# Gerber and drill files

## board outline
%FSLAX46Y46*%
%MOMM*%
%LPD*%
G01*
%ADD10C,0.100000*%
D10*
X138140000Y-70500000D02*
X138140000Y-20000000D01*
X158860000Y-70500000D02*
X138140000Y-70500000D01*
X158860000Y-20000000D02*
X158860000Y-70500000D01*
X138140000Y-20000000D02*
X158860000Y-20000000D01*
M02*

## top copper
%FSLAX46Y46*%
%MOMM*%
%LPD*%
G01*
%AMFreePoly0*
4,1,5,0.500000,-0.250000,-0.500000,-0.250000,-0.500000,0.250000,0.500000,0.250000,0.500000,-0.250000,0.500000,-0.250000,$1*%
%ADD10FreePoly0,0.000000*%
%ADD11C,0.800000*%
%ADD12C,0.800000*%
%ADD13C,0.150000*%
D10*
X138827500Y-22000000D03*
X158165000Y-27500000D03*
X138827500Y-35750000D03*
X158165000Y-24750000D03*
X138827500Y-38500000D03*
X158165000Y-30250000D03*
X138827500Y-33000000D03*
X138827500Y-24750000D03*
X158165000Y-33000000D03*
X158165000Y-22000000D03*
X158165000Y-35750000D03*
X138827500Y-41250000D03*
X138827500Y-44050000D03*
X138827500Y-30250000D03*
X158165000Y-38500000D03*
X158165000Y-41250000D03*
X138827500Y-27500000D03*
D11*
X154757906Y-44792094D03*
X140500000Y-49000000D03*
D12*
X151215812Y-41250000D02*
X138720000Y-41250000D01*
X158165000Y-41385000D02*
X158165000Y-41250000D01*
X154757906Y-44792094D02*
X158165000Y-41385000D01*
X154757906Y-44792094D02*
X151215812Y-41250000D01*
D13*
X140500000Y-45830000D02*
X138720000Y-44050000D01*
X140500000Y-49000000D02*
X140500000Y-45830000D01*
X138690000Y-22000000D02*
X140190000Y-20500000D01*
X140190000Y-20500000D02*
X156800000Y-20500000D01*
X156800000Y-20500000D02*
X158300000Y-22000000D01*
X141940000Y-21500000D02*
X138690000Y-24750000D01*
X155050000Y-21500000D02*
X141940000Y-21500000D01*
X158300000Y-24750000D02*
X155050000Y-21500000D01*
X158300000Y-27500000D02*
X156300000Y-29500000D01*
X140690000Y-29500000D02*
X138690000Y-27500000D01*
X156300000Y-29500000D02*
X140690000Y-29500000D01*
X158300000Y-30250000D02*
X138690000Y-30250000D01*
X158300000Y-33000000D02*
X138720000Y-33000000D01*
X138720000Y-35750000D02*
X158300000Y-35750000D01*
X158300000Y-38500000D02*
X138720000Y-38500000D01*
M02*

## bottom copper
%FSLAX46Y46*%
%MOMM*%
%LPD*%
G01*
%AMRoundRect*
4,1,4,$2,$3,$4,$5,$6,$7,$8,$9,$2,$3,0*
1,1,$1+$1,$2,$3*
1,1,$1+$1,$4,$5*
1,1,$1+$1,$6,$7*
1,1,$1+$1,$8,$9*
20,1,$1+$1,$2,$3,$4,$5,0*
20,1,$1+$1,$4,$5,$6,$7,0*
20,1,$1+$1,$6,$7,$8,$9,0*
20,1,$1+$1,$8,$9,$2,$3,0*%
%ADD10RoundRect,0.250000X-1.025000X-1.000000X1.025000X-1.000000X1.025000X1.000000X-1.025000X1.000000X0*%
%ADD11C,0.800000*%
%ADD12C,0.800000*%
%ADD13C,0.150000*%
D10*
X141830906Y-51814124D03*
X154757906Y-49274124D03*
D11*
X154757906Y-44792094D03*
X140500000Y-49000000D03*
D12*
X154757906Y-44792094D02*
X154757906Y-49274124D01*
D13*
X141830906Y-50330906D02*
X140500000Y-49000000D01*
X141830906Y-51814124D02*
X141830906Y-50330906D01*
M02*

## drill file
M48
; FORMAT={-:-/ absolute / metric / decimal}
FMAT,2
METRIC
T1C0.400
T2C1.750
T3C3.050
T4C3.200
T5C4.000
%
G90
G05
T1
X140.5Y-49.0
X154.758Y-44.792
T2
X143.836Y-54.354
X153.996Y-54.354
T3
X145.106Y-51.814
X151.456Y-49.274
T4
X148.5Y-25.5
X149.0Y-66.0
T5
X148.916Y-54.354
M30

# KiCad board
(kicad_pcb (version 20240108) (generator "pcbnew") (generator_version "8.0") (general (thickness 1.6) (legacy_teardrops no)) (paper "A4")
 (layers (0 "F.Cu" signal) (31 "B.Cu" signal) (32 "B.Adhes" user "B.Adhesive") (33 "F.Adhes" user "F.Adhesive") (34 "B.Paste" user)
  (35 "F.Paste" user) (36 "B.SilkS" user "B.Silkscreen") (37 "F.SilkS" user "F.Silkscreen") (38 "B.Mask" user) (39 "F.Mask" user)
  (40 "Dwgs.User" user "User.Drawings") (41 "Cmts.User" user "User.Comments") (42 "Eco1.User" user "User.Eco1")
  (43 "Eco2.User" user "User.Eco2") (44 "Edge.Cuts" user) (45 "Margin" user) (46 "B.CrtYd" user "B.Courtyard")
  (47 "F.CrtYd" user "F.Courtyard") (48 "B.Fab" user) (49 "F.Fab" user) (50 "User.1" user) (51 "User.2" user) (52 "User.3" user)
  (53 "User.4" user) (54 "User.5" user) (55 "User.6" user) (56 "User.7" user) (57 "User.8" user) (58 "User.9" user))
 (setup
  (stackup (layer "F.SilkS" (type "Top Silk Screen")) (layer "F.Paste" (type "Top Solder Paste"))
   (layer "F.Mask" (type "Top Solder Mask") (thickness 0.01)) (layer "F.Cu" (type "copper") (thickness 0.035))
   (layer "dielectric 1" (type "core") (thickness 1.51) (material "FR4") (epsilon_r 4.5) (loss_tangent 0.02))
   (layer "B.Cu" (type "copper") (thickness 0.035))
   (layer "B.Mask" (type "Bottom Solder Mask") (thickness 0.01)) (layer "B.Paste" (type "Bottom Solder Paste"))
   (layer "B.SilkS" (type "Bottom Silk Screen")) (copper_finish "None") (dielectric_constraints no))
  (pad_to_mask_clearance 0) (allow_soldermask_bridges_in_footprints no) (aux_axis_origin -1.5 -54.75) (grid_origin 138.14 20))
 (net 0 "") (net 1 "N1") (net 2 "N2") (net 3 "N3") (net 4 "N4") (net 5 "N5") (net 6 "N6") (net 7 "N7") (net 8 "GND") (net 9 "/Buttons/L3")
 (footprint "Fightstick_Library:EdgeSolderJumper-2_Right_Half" (layer "F.Cu") (at 138.1775 22)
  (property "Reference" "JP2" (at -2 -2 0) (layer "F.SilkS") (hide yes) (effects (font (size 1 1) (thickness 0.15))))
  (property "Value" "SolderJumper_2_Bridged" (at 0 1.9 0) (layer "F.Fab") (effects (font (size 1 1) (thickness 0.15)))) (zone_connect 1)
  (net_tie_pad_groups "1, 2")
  (pad "2" smd custom (at 0.65 0) (size 1 0.5) (layers "F.Cu" "F.Mask") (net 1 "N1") (zone_connect 2) (thermal_bridge_angle 45)
   (options (clearance outline) (anchor rect)) (primitives)))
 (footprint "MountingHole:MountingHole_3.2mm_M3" (layer "F.Cu") (at 149 66)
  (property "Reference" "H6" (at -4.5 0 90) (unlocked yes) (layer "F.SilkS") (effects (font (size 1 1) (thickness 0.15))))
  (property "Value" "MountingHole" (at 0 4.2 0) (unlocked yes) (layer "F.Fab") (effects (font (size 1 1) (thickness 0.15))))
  (pad "" np_thru_hole circle (at 0 0) (size 3.2 3.2) (drill 3.2) (layers "*.Cu" "*.Mask")))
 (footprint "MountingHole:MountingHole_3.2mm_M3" (layer "F.Cu") (at 148.5 25.5)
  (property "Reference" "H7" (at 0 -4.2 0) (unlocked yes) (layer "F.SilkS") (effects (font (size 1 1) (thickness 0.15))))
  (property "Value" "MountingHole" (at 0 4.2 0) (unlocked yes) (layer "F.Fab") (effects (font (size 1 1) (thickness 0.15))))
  (pad "" np_thru_hole circle (at 0 0) (size 3.2 3.2) (drill 3.2) (layers "*.Cu" "*.Mask")))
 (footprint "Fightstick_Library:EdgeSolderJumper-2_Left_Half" (layer "F.Cu") (at 158.815 27.5)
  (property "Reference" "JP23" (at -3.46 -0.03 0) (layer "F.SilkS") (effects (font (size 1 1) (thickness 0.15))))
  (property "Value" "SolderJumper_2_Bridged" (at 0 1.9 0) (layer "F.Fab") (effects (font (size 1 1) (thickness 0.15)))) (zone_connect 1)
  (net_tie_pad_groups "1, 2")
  (pad "1" smd custom (at -0.65 0) (size 1 0.5) (layers "F.Cu" "F.Mask") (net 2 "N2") (zone_connect 2) (thermal_bridge_angle 45)
   (options (clearance outline) (anchor rect)) (primitives)))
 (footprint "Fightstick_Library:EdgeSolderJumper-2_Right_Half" (layer "F.Cu") (at 138.1775 35.75)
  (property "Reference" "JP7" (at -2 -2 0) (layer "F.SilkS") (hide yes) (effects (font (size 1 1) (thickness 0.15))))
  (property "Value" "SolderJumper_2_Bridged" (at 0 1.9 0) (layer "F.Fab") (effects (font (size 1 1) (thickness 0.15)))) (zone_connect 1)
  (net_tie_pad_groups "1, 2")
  (pad "2" smd custom (at 0.65 0) (size 1 0.5) (layers "F.Cu" "F.Mask") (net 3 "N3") (zone_connect 2) (thermal_bridge_angle 45)
   (options (clearance outline) (anchor rect)) (primitives)))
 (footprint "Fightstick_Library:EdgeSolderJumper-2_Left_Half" (layer "F.Cu") (at 158.815 24.75)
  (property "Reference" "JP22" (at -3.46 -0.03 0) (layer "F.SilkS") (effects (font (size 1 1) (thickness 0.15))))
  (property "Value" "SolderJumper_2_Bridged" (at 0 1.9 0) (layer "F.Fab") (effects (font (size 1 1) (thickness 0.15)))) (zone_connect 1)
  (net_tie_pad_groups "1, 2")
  (pad "1" smd custom (at -0.65 0) (size 1 0.5) (layers "F.Cu" "F.Mask") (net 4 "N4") (zone_connect 2) (thermal_bridge_angle 45)
   (options (clearance outline) (anchor rect)) (primitives)))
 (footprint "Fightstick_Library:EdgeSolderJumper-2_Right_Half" (layer "F.Cu") (at 138.1775 38.5)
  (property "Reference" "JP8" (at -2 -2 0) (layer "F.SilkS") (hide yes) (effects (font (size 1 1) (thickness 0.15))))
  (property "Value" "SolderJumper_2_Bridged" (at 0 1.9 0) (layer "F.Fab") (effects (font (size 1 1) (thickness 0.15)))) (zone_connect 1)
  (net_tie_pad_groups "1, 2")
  (pad "2" smd custom (at 0.65 0) (size 1 0.5) (layers "F.Cu" "F.Mask") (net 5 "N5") (zone_connect 2) (thermal_bridge_angle 45)
   (options (clearance outline) (anchor rect)) (primitives)))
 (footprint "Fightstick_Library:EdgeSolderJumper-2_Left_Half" (layer "F.Cu") (at 158.815 30.25)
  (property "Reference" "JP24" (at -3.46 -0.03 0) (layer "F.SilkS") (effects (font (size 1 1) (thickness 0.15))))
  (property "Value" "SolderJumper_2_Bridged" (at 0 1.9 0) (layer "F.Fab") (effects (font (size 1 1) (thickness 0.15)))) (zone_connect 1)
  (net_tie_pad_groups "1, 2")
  (pad "1" smd custom (at -0.65 0) (size 1 0.5) (layers "F.Cu" "F.Mask") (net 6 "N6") (zone_connect 2) (thermal_bridge_angle 45)
   (options (clearance outline) (anchor rect)) (primitives)))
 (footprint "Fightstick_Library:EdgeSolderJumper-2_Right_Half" (layer "F.Cu") (at 138.1775 33)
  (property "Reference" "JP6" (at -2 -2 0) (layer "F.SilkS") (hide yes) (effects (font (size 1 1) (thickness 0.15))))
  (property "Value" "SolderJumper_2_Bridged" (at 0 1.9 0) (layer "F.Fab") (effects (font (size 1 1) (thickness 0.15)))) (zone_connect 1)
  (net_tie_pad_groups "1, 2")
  (pad "2" smd custom (at 0.65 0) (size 1 0.5) (layers "F.Cu" "F.Mask") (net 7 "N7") (zone_connect 2) (thermal_bridge_angle 45)
   (options (clearance outline) (anchor rect)) (primitives)))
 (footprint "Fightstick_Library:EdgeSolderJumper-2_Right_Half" (layer "F.Cu") (at 138.1775 24.75)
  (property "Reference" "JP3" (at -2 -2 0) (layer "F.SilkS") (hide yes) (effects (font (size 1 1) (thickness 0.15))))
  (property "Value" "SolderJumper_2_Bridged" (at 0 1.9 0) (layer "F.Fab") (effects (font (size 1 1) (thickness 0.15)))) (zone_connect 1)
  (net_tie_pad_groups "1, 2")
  (pad "2" smd custom (at 0.65 0) (size 1 0.5) (layers "F.Cu" "F.Mask") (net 4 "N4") (zone_connect 2) (thermal_bridge_angle 45)
   (options (clearance outline) (anchor rect)) (primitives)))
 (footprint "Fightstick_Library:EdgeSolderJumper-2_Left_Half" (layer "F.Cu") (at 158.815 33)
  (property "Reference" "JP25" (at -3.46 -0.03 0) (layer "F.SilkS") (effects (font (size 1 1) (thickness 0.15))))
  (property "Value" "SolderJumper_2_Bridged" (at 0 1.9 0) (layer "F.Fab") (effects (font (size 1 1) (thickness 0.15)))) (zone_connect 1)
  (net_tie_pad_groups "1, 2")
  (pad "1" smd custom (at -0.65 0) (size 1 0.5) (layers "F.Cu" "F.Mask") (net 7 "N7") (zone_connect 2) (thermal_bridge_angle 45)
   (options (clearance outline) (anchor rect)) (primitives)))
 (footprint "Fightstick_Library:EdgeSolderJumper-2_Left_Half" (layer "F.Cu") (at 158.815 22)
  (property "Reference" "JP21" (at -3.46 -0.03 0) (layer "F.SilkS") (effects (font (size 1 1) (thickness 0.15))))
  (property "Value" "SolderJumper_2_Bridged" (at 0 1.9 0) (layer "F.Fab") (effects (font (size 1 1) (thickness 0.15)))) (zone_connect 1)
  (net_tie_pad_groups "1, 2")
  (pad "1" smd custom (at -0.65 0) (size 1 0.5) (layers "F.Cu" "F.Mask") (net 1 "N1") (zone_connect 2) (thermal_bridge_angle 45)
   (options (clearance outline) (anchor rect)) (primitives)))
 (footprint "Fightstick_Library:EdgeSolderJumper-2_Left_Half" (layer "F.Cu") (at 158.815 35.75)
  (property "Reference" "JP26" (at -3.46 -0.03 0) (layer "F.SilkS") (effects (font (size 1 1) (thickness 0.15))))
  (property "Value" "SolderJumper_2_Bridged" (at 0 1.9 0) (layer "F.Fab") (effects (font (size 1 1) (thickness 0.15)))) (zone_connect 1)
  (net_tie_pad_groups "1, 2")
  (pad "1" smd custom (at -0.65 0) (size 1 0.5) (layers "F.Cu" "F.Mask") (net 3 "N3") (zone_connect 2) (thermal_bridge_angle 45)
   (options (clearance outline) (anchor rect)) (primitives)))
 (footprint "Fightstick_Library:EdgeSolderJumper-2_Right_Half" (layer "F.Cu") (at 138.1775 41.25)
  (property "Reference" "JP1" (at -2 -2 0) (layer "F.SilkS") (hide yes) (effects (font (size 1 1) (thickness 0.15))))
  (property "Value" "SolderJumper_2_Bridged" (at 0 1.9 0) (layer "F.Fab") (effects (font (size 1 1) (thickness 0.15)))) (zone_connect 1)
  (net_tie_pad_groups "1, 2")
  (pad "2" smd custom (at 0.65 0) (size 1 0.5) (layers "F.Cu" "F.Mask") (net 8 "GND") (zone_connect 2) (thermal_bridge_angle 45)
   (options (clearance outline) (anchor rect)) (primitives)))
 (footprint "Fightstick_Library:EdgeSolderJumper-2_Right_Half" (layer "F.Cu") (at 138.1775 44.05)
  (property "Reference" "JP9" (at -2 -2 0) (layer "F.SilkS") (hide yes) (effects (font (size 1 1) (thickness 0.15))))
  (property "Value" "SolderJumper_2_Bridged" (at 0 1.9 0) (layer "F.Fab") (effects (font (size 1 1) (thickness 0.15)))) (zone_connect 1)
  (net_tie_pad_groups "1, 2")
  (pad "2" smd custom (at 0.65 0) (size 1 0.5) (layers "F.Cu" "F.Mask") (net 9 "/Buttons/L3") (zone_connect 2) (thermal_bridge_angle 45)
   (options (clearance outline) (anchor rect)) (primitives)))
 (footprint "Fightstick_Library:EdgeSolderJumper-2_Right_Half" (layer "F.Cu") (at 138.1775 30.25)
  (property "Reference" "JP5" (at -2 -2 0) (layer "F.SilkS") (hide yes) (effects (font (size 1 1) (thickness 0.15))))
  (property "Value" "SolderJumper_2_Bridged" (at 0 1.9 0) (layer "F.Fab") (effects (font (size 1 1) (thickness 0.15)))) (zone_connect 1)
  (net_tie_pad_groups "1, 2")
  (pad "2" smd custom (at 0.65 0) (size 1 0.5) (layers "F.Cu" "F.Mask") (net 6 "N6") (zone_connect 2) (thermal_bridge_angle 45)
   (options (clearance outline) (anchor rect)) (primitives)))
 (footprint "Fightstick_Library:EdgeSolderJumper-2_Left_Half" (layer "F.Cu") (at 158.815 38.5)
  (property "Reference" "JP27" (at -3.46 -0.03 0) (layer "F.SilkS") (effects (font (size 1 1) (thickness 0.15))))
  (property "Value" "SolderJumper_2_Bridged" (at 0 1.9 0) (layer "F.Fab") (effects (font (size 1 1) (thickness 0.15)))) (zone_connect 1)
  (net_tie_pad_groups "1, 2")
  (pad "1" smd custom (at -0.65 0) (size 1 0.5) (layers "F.Cu" "F.Mask") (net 5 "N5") (zone_connect 2) (thermal_bridge_angle 45)
   (options (clearance outline) (anchor rect)) (primitives)))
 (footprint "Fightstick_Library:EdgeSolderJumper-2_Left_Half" (layer "F.Cu") (at 158.815 41.25)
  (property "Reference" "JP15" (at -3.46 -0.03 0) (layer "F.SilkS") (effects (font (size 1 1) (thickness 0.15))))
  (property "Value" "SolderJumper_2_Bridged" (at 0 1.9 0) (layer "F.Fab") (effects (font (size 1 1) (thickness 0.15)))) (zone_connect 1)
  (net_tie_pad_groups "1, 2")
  (pad "1" smd custom (at -0.65 0) (size 1 0.5) (layers "F.Cu" "F.Mask") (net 8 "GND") (zone_connect 2) (thermal_bridge_angle 45)
   (options (clearance outline) (anchor rect)) (primitives)))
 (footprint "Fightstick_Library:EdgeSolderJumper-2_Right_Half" (layer "F.Cu") (at 138.1775 27.5)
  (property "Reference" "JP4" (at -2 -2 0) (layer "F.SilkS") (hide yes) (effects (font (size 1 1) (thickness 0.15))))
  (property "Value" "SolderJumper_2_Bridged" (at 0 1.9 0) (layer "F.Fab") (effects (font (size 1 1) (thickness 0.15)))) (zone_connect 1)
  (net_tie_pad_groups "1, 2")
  (pad "2" smd custom (at 0.65 0) (size 1 0.5) (layers "F.Cu" "F.Mask") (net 2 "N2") (zone_connect 2) (thermal_bridge_angle 45)
   (options (clearance outline) (anchor rect)) (primitives)))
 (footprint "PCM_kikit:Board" (layer "F.Cu") (at 150.375 20)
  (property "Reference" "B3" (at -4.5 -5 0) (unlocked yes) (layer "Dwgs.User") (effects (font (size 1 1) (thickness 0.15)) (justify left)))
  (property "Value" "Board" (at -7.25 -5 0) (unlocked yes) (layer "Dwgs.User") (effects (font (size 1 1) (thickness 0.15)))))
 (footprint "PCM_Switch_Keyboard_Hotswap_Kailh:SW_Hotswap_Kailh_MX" (layer "F.Cu") (at 148.915906 54.354124)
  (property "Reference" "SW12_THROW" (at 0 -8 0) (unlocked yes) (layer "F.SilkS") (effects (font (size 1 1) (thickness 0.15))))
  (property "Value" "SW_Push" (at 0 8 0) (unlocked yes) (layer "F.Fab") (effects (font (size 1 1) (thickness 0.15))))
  (pad "" np_thru_hole circle (at -5.08 0) (size 1.75 1.75) (drill 1.75) (layers "*.Cu" "*.Mask"))
  (pad "" np_thru_hole circle (at -3.81 -2.54) (size 3.05 3.05) (drill 3.05) (layers "*.Cu" "*.Mask"))
  (pad "" np_thru_hole circle (at 0 0) (size 4 4) (drill 4) (layers "*.Cu" "*.Mask"))
  (pad "" np_thru_hole circle (at 2.54 -5.08) (size 3.05 3.05) (drill 3.05) (layers "*.Cu" "*.Mask"))
  (pad "" np_thru_hole circle (at 5.08 0) (size 1.75 1.75) (drill 1.75) (layers "*.Cu" "*.Mask"))
  (pad "1" smd roundrect (at -7.085 -2.54) (size 2.55 2.5) (layers "B.Cu" "B.Paste" "B.Mask") (roundrect_rratio 0.1) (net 9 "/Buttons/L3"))
  (pad "2" smd roundrect (at 5.842 -5.08) (size 2.55 2.5) (layers "B.Cu" "B.Paste" "B.Mask") (roundrect_rratio 0.1) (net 8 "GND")))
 (gr_line (start 138.14 70.5) (end 138.14 20) (stroke (width 0.1) (type default)) (layer "Edge.Cuts"))
 (gr_line (start 158.86 70.5) (end 138.14 70.5) (stroke (width 0.1) (type default)) (layer "Edge.Cuts"))
 (gr_line (start 158.86 20) (end 158.86 70.5) (stroke (width 0.1) (type default)) (layer "Edge.Cuts"))
 (gr_line (start 138.14 20) (end 158.86 20) (stroke (width 0.1) (type default)) (layer "Edge.Cuts"))
 (segment (start 151.215812 41.25) (end 138.72 41.25) (width 0.8) (layer "F.Cu") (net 8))
 (segment (start 158.165 41.385) (end 158.165 41.25) (width 0.8) (layer "F.Cu") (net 8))
 (segment (start 154.757906 44.792094) (end 158.165 41.385) (width 0.8) (layer "F.Cu") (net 8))
 (segment (start 154.757906 44.792094) (end 151.215812 41.25) (width 0.8) (layer "F.Cu") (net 8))
 (via (at 154.757906 44.792094) (size 0.8) (drill 0.4) (layers "F.Cu" "B.Cu") (free yes) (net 8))
 (segment (start 154.757906 44.792094) (end 154.757906 49.274124) (width 0.8) (layer "B.Cu") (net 8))
 (segment (start 140.5 45.83) (end 138.72 44.05) (width 0.15) (layer "F.Cu") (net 9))
 (segment (start 140.5 49) (end 140.5 45.83) (width 0.15) (layer "F.Cu") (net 9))
 (via (at 140.5 49) (size 0.8) (drill 0.4) (layers "F.Cu" "B.Cu") (free yes) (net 9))
 (segment (start 141.830906 50.330906) (end 140.5 49) (width 0.15) (layer "B.Cu") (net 9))
 (segment (start 141.830906 51.814124) (end 141.830906 50.330906) (width 0.15) (layer "B.Cu") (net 9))
 (segment (start 138.69 22) (end 140.19 20.5) (width 0.15) (layer "F.Cu") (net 1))
 (segment (start 140.19 20.5) (end 156.8 20.5) (width 0.15) (layer "F.Cu") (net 1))
 (segment (start 156.8 20.5) (end 158.3 22) (width 0.15) (layer "F.Cu") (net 1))
 (segment (start 141.94 21.5) (end 138.69 24.75) (width 0.15) (layer "F.Cu") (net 4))
 (segment (start 155.05 21.5) (end 141.94 21.5) (width 0.15) (layer "F.Cu") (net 4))
 (segment (start 158.3 24.75) (end 155.05 21.5) (width 0.15) (layer "F.Cu") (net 4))
 (segment (start 158.3 27.5) (end 156.3 29.5) (width 0.15) (layer "F.Cu") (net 2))
 (segment (start 140.69 29.5) (end 138.69 27.5) (width 0.15) (layer "F.Cu") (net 2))
 (segment (start 156.3 29.5) (end 140.69 29.5) (width 0.15) (layer "F.Cu") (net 2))
 (segment (start 158.3 30.25) (end 138.69 30.25) (width 0.15) (layer "F.Cu") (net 6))
 (segment (start 158.3 33) (end 138.72 33) (width 0.15) (layer "F.Cu") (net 7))
 (segment (start 138.72 35.75) (end 158.3 35.75) (width 0.15) (layer "F.Cu") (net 3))
 (segment (start 158.3 38.5) (end 138.72 38.5) (width 0.15) (layer "F.Cu") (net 5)))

